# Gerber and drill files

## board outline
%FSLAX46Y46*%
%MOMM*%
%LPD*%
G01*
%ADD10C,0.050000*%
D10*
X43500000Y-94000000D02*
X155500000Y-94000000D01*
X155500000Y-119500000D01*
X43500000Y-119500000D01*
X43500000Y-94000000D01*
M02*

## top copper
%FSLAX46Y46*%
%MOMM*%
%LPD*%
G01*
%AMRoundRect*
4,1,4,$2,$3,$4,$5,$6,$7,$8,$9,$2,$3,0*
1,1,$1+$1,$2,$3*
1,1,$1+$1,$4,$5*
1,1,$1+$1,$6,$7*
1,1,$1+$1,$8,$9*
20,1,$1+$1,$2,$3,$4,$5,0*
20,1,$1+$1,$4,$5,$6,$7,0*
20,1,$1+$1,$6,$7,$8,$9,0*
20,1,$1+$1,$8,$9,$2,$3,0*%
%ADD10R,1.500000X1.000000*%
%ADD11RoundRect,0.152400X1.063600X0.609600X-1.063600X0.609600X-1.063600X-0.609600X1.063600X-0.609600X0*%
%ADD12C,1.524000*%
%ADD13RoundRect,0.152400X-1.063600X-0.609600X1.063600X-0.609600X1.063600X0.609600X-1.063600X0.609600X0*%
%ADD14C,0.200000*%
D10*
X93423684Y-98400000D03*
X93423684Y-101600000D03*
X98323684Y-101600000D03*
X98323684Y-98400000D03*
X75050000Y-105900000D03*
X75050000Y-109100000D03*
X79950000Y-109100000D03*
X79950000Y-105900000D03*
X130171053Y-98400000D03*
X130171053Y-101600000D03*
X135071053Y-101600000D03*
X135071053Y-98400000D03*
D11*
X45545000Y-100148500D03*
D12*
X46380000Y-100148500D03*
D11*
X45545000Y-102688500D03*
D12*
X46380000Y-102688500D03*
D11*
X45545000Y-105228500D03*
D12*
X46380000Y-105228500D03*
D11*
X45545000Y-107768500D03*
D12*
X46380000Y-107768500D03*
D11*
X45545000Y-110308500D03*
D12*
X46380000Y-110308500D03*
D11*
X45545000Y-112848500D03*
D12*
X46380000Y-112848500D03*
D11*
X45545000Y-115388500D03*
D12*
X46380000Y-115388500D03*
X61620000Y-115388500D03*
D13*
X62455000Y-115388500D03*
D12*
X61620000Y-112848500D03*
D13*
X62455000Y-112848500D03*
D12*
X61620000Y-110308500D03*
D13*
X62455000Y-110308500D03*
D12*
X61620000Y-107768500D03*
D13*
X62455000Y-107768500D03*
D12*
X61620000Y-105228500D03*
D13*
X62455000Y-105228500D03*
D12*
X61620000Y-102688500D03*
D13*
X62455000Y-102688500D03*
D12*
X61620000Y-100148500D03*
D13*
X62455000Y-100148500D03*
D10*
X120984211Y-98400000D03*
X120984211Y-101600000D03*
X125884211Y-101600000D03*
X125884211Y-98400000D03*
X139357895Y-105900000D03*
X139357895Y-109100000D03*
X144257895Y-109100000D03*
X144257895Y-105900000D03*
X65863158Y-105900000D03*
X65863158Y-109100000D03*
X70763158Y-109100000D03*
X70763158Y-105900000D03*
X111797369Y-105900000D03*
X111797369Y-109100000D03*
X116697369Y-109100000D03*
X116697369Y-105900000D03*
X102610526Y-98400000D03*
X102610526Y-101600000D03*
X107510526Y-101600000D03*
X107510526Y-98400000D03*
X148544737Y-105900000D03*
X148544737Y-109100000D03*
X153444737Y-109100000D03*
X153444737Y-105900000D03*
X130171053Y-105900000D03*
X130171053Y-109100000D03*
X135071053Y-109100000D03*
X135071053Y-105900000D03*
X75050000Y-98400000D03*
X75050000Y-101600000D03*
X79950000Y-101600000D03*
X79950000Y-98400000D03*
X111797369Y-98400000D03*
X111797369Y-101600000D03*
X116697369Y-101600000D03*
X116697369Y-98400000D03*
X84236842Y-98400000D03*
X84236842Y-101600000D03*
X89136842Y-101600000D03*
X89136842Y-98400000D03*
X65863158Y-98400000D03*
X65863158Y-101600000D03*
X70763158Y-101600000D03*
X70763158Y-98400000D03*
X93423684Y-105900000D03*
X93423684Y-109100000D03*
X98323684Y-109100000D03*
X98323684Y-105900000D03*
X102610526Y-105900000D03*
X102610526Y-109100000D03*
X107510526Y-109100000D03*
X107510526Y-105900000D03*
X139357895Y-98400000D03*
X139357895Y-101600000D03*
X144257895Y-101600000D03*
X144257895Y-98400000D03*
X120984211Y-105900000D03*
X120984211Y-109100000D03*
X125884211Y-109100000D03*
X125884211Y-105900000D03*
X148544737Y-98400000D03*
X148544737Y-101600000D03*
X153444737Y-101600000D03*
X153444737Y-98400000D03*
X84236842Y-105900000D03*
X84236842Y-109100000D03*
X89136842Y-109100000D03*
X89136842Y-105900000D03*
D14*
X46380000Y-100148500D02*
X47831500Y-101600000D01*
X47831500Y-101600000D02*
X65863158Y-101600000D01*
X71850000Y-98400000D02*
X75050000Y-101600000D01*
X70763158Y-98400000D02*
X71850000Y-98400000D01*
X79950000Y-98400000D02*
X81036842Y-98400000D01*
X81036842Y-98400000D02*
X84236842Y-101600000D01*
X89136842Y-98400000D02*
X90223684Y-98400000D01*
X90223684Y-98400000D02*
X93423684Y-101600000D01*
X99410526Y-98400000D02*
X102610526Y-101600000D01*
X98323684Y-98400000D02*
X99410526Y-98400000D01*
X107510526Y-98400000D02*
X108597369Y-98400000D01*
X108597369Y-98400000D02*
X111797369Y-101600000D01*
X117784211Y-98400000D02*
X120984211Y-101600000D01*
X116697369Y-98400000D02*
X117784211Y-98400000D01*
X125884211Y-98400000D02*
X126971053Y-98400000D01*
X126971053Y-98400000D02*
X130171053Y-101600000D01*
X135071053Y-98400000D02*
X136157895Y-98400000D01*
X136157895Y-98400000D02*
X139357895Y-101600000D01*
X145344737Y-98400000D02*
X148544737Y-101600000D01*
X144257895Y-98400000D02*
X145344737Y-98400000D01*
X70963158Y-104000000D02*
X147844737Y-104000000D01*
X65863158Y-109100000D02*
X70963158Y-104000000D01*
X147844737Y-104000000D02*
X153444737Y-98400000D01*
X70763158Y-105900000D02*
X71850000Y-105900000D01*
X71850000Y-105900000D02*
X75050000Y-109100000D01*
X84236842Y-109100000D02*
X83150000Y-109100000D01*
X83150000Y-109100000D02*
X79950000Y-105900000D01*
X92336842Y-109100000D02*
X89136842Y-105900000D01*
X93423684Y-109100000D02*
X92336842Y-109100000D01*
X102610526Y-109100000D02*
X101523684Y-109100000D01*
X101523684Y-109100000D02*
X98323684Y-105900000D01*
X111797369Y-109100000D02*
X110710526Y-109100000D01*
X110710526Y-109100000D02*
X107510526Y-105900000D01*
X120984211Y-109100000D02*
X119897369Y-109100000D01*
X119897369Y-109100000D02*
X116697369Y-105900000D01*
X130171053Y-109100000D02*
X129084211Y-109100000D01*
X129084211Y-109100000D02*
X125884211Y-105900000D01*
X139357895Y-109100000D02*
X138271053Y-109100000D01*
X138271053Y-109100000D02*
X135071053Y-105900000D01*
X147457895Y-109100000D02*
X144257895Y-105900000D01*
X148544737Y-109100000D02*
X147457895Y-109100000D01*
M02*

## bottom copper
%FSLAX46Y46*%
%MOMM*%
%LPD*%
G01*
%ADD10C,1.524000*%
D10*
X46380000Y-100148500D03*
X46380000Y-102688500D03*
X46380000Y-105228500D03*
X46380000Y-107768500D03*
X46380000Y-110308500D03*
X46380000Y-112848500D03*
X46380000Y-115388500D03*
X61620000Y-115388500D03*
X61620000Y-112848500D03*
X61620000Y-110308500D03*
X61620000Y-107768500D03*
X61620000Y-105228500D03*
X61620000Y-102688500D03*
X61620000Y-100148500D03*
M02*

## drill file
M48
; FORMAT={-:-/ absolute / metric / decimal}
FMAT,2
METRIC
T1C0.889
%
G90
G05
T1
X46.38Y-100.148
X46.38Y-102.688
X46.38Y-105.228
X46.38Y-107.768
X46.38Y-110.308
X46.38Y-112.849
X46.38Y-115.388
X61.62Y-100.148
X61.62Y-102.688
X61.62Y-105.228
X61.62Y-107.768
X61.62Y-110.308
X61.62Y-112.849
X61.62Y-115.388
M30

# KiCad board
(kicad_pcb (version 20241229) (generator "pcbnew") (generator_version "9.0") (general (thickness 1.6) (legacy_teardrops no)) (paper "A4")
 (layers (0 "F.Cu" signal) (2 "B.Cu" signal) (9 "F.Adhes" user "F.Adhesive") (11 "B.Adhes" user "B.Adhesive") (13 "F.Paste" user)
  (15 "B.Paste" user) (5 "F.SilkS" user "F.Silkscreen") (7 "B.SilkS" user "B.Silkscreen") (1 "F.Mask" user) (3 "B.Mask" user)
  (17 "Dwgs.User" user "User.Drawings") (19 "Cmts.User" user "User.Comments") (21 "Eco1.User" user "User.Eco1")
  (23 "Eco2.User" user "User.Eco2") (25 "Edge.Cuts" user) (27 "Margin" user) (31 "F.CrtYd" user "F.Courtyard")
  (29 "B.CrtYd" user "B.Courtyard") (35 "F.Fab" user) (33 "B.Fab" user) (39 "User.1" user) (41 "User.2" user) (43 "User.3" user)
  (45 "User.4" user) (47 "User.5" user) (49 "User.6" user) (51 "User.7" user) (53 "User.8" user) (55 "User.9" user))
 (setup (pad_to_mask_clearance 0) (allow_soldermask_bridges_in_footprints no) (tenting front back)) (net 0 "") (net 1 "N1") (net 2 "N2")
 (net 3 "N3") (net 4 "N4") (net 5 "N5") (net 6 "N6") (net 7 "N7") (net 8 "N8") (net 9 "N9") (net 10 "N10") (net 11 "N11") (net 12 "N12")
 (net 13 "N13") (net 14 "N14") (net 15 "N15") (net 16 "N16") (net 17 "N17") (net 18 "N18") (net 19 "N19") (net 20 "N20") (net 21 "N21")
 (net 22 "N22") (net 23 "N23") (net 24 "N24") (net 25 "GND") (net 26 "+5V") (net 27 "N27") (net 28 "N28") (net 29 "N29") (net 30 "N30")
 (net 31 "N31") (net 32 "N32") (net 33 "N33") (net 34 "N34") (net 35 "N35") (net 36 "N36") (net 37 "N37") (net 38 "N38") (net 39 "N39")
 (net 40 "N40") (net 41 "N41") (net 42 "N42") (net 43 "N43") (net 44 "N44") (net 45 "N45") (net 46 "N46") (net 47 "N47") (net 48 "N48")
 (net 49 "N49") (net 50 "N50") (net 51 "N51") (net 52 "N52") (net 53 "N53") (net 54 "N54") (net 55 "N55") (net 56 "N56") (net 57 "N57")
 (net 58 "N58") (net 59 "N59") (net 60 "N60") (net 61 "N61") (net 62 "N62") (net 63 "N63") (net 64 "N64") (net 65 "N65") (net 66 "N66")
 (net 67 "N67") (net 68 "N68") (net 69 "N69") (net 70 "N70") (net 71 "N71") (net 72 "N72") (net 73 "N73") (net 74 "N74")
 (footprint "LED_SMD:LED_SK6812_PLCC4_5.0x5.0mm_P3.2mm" (layer "F.Cu") (at 95.873684 100)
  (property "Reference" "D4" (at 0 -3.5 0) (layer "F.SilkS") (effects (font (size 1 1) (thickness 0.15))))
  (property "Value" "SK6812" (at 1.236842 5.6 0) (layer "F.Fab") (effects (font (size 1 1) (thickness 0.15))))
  (pad "1" smd rect (at -2.45 -1.6 180) (size 1.5 1) (layers "F.Cu" "F.Mask" "F.Paste") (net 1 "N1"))
  (pad "2" smd rect (at -2.45 1.6 180) (size 1.5 1) (layers "F.Cu" "F.Mask" "F.Paste") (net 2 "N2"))
  (pad "3" smd rect (at 2.45 1.6 180) (size 1.5 1) (layers "F.Cu" "F.Mask" "F.Paste") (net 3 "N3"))
  (pad "4" smd rect (at 2.45 -1.6 180) (size 1.5 1) (layers "F.Cu" "F.Mask" "F.Paste") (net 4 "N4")))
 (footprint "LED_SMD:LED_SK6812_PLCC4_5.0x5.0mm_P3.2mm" (layer "F.Cu") (at 77.5 107.5)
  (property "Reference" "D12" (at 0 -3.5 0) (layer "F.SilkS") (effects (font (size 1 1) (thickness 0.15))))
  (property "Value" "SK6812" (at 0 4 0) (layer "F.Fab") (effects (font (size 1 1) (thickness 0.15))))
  (pad "1" smd rect (at -2.45 -1.6 180) (size 1.5 1) (layers "F.Cu" "F.Mask" "F.Paste") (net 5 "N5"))
  (pad "2" smd rect (at -2.45 1.6 180) (size 1.5 1) (layers "F.Cu" "F.Mask" "F.Paste") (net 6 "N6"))
  (pad "3" smd rect (at 2.45 1.6 180) (size 1.5 1) (layers "F.Cu" "F.Mask" "F.Paste") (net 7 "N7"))
  (pad "4" smd rect (at 2.45 -1.6 180) (size 1.5 1) (layers "F.Cu" "F.Mask" "F.Paste") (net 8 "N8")))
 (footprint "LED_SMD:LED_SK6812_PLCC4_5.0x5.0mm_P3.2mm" (layer "F.Cu") (at 132.621053 100)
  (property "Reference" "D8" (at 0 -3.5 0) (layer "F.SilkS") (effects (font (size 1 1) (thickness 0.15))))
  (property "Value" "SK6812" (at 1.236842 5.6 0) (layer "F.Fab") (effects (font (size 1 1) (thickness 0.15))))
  (pad "1" smd rect (at -2.45 -1.6 180) (size 1.5 1) (layers "F.Cu" "F.Mask" "F.Paste") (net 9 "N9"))
  (pad "2" smd rect (at -2.45 1.6 180) (size 1.5 1) (layers "F.Cu" "F.Mask" "F.Paste") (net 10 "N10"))
  (pad "3" smd rect (at 2.45 1.6 180) (size 1.5 1) (layers "F.Cu" "F.Mask" "F.Paste") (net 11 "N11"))
  (pad "4" smd rect (at 2.45 -1.6 180) (size 1.5 1) (layers "F.Cu" "F.Mask" "F.Paste") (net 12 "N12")))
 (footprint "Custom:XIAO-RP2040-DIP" (layer "F.Cu") (at 54 107.7685)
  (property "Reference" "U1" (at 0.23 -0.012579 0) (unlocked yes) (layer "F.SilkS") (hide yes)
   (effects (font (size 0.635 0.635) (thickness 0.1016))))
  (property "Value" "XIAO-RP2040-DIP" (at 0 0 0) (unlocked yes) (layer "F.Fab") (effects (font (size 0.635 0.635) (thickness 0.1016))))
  (pad "1" smd roundrect (at -8.455 -7.62 180) (size 2.432 1.524) (layers "F.Cu" "F.Mask") (roundrect_rratio 0.1) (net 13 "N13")
   (thermal_bridge_angle 45))
  (pad "1" thru_hole circle (at -7.62 -7.62 180) (size 1.524 1.524) (drill 0.889) (layers "*.Cu" "*.Mask") (remove_unused_layers no)
   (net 13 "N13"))
  (pad "2" smd roundrect (at -8.455 -5.08 180) (size 2.432 1.524) (layers "F.Cu" "F.Mask") (roundrect_rratio 0.1) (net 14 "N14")
   (thermal_bridge_angle 45))
  (pad "2" thru_hole circle (at -7.62 -5.08 180) (size 1.524 1.524) (drill 0.889) (layers "*.Cu" "*.Mask") (remove_unused_layers no)
   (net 14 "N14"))
  (pad "3" smd roundrect (at -8.455 -2.54 180) (size 2.432 1.524) (layers "F.Cu" "F.Mask") (roundrect_rratio 0.1) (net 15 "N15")
   (thermal_bridge_angle 45))
  (pad "3" thru_hole circle (at -7.62 -2.54 180) (size 1.524 1.524) (drill 0.889) (layers "*.Cu" "*.Mask") (remove_unused_layers no)
   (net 15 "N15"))
  (pad "4" smd roundrect (at -8.455 0 180) (size 2.432 1.524) (layers "F.Cu" "F.Mask") (roundrect_rratio 0.1) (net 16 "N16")
   (thermal_bridge_angle 45))
  (pad "4" thru_hole circle (at -7.62 0 180) (size 1.524 1.524) (drill 0.889) (layers "*.Cu" "*.Mask") (remove_unused_layers no)
   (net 16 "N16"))
  (pad "5" smd roundrect (at -8.455 2.54 180) (size 2.432 1.524) (layers "F.Cu" "F.Mask") (roundrect_rratio 0.1) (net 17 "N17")
   (thermal_bridge_angle 45))
  (pad "5" thru_hole circle (at -7.62 2.54 180) (size 1.524 1.524) (drill 0.889) (layers "*.Cu" "*.Mask") (remove_unused_layers no)
   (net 17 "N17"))
  (pad "6" smd roundrect (at -8.455 5.08 180) (size 2.432 1.524) (layers "F.Cu" "F.Mask") (roundrect_rratio 0.1) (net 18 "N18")
   (thermal_bridge_angle 45))
  (pad "6" thru_hole circle (at -7.62 5.08 180) (size 1.524 1.524) (drill 0.889) (layers "*.Cu" "*.Mask") (remove_unused_layers no)
   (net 18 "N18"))
  (pad "7" smd roundrect (at -8.455 7.62 180) (size 2.432 1.524) (layers "F.Cu" "F.Mask") (roundrect_rratio 0.1) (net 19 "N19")
   (thermal_bridge_angle 45))
  (pad "7" thru_hole circle (at -7.62 7.62 180) (size 1.524 1.524) (drill 0.889) (layers "*.Cu" "*.Mask") (remove_unused_layers no)
   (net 19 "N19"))
  (pad "8" thru_hole circle (at 7.62 7.62) (size 1.524 1.524) (drill 0.889) (layers "*.Cu" "*.Mask") (remove_unused_layers no)
   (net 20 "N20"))
  (pad "8" smd roundrect (at 8.455 7.62) (size 2.432 1.524) (layers "F.Cu" "F.Mask") (roundrect_rratio 0.1) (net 20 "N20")
   (thermal_bridge_angle 45))
  (pad "9" thru_hole circle (at 7.62 5.08) (size 1.524 1.524) (drill 0.889) (layers "*.Cu" "*.Mask") (remove_unused_layers no)
   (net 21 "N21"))
  (pad "9" smd roundrect (at 8.455 5.08) (size 2.432 1.524) (layers "F.Cu" "F.Mask") (roundrect_rratio 0.1) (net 21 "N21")
   (thermal_bridge_angle 45))
  (pad "10" thru_hole circle (at 7.62 2.54) (size 1.524 1.524) (drill 0.889) (layers "*.Cu" "*.Mask") (remove_unused_layers no)
   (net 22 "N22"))
  (pad "10" smd roundrect (at 8.455 2.54) (size 2.432 1.524) (layers "F.Cu" "F.Mask") (roundrect_rratio 0.1) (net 22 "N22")
   (thermal_bridge_angle 45))
  (pad "11" thru_hole circle (at 7.62 0) (size 1.524 1.524) (drill 0.889) (layers "*.Cu" "*.Mask") (remove_unused_layers no) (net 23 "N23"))
  (pad "11" smd roundrect (at 8.455 0) (size 2.432 1.524) (layers "F.Cu" "F.Mask") (roundrect_rratio 0.1) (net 23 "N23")
   (thermal_bridge_angle 45))
  (pad "12" thru_hole circle (at 7.62 -2.54) (size 1.524 1.524) (drill 0.889) (layers "*.Cu" "*.Mask") (remove_unused_layers no)
   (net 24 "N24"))
  (pad "12" smd roundrect (at 8.455 -2.54) (size 2.432 1.524) (layers "F.Cu" "F.Mask") (roundrect_rratio 0.1) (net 24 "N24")
   (thermal_bridge_angle 45))
  (pad "13" thru_hole circle (at 7.62 -5.08) (size 1.524 1.524) (drill 0.889) (layers "*.Cu" "*.Mask") (remove_unused_layers no)
   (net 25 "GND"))
  (pad "13" smd roundrect (at 8.455 -5.08) (size 2.432 1.524) (layers "F.Cu" "F.Mask") (roundrect_rratio 0.1) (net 25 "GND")
   (thermal_bridge_angle 45))
  (pad "14" thru_hole circle (at 7.62 -7.62) (size 1.524 1.524) (drill 0.889) (layers "*.Cu" "*.Mask") (remove_unused_layers no)
   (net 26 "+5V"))
  (pad "14" smd roundrect (at 8.455 -7.62) (size 2.432 1.524) (layers "F.Cu" "F.Mask") (roundrect_rratio 0.1) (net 26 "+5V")
   (thermal_bridge_angle 45)))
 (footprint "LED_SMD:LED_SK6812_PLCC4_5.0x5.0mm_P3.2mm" (layer "F.Cu") (at 123.434211 100)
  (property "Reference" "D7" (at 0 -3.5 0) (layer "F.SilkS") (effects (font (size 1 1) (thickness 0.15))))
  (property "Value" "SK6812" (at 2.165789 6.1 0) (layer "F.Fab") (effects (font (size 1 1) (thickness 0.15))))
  (pad "1" smd rect (at -2.45 -1.6 180) (size 1.5 1) (layers "F.Cu" "F.Mask" "F.Paste") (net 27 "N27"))
  (pad "2" smd rect (at -2.45 1.6 180) (size 1.5 1) (layers "F.Cu" "F.Mask" "F.Paste") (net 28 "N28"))
  (pad "3" smd rect (at 2.45 1.6 180) (size 1.5 1) (layers "F.Cu" "F.Mask" "F.Paste") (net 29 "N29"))
  (pad "4" smd rect (at 2.45 -1.6 180) (size 1.5 1) (layers "F.Cu" "F.Mask" "F.Paste") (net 10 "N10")))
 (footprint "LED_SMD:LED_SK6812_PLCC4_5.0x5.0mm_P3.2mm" (layer "F.Cu") (at 141.807895 107.5)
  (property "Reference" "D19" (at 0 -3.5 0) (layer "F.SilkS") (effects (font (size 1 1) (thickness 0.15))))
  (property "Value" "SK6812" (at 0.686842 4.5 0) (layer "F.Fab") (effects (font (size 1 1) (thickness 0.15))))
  (pad "1" smd rect (at -2.45 -1.6 180) (size 1.5 1) (layers "F.Cu" "F.Mask" "F.Paste") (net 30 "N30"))
  (pad "2" smd rect (at -2.45 1.6 180) (size 1.5 1) (layers "F.Cu" "F.Mask" "F.Paste") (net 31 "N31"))
  (pad "3" smd rect (at 2.45 1.6 180) (size 1.5 1) (layers "F.Cu" "F.Mask" "F.Paste") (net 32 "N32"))
  (pad "4" smd rect (at 2.45 -1.6 180) (size 1.5 1) (layers "F.Cu" "F.Mask" "F.Paste") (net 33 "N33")))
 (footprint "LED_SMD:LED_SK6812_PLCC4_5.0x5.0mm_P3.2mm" (layer "F.Cu") (at 68.313158 107.5)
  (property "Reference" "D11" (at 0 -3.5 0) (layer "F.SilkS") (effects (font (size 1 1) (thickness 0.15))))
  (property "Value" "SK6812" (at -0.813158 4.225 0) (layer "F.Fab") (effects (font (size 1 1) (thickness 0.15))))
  (pad "1" smd rect (at -2.45 -1.6 180) (size 1.5 1) (layers "F.Cu" "F.Mask" "F.Paste") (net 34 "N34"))
  (pad "2" smd rect (at -2.45 1.6 180) (size 1.5 1) (layers "F.Cu" "F.Mask" "F.Paste") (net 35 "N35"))
  (pad "3" smd rect (at 2.45 1.6 180) (size 1.5 1) (layers "F.Cu" "F.Mask" "F.Paste") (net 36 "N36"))
  (pad "4" smd rect (at 2.45 -1.6 180) (size 1.5 1) (layers "F.Cu" "F.Mask" "F.Paste") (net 6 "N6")))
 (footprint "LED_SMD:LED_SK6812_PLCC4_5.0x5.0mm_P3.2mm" (layer "F.Cu") (at 114.247369 107.5)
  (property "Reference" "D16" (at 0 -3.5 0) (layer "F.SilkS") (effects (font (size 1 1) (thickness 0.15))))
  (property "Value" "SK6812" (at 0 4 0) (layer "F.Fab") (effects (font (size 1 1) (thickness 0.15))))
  (pad "1" smd rect (at -2.45 -1.6 180) (size 1.5 1) (layers "F.Cu" "F.Mask" "F.Paste") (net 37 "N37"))
  (pad "2" smd rect (at -2.45 1.6 180) (size 1.5 1) (layers "F.Cu" "F.Mask" "F.Paste") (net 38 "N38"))
  (pad "3" smd rect (at 2.45 1.6 180) (size 1.5 1) (layers "F.Cu" "F.Mask" "F.Paste") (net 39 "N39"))
  (pad "4" smd rect (at 2.45 -1.6 180) (size 1.5 1) (layers "F.Cu" "F.Mask" "F.Paste") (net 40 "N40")))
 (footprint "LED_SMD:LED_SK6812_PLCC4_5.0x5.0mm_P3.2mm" (layer "F.Cu") (at 105.060526 100)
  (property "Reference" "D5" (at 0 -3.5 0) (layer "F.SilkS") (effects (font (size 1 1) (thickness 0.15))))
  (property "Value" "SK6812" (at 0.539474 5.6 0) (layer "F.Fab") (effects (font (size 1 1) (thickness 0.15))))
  (pad "1" smd rect (at -2.45 -1.6 180) (size 1.5 1) (layers "F.Cu" "F.Mask" "F.Paste") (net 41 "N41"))
  (pad "2" smd rect (at -2.45 1.6 180) (size 1.5 1) (layers "F.Cu" "F.Mask" "F.Paste") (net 4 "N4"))
  (pad "3" smd rect (at 2.45 1.6 180) (size 1.5 1) (layers "F.Cu" "F.Mask" "F.Paste") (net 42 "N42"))
  (pad "4" smd rect (at 2.45 -1.6 180) (size 1.5 1) (layers "F.Cu" "F.Mask" "F.Paste") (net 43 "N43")))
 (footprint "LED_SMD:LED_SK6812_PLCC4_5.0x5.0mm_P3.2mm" (layer "F.Cu") (at 150.994737 107.5)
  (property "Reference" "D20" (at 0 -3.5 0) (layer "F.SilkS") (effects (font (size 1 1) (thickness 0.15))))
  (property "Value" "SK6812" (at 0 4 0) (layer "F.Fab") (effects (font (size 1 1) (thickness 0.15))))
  (pad "1" smd rect (at -2.45 -1.6 180) (size 1.5 1) (layers "F.Cu" "F.Mask" "F.Paste") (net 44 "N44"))
  (pad "2" smd rect (at -2.45 1.6 180) (size 1.5 1) (layers "F.Cu" "F.Mask" "F.Paste") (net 33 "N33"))
  (pad "3" smd rect (at 2.45 1.6 180) (size 1.5 1) (layers "F.Cu" "F.Mask" "F.Paste") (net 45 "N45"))
  (pad "4" smd rect (at 2.45 -1.6 180) (size 1.5 1) (layers "F.Cu" "F.Mask" "F.Paste") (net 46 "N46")))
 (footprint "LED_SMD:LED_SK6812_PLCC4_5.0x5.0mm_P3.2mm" (layer "F.Cu") (at 132.621053 107.5)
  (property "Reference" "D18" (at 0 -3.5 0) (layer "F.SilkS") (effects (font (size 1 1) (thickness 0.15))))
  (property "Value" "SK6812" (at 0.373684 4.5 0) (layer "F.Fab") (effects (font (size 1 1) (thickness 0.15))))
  (pad "1" smd rect (at -2.45 -1.6 180) (size 1.5 1) (layers "F.Cu" "F.Mask" "F.Paste") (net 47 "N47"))
  (pad "2" smd rect (at -2.45 1.6 180) (size 1.5 1) (layers "F.Cu" "F.Mask" "F.Paste") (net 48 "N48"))
  (pad "3" smd rect (at 2.45 1.6 180) (size 1.5 1) (layers "F.Cu" "F.Mask" "F.Paste") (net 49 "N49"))
  (pad "4" smd rect (at 2.45 -1.6 180) (size 1.5 1) (layers "F.Cu" "F.Mask" "F.Paste") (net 31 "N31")))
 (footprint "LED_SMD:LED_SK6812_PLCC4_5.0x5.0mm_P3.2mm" (layer "F.Cu") (at 77.5 100)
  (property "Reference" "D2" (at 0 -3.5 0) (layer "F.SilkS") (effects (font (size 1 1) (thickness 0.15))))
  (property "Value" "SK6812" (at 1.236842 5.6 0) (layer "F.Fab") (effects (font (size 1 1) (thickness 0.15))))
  (pad "1" smd rect (at -2.45 -1.6 180) (size 1.5 1) (layers "F.Cu" "F.Mask" "F.Paste") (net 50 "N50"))
  (pad "2" smd rect (at -2.45 1.6 180) (size 1.5 1) (layers "F.Cu" "F.Mask" "F.Paste") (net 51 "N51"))
  (pad "3" smd rect (at 2.45 1.6 180) (size 1.5 1) (layers "F.Cu" "F.Mask" "F.Paste") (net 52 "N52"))
  (pad "4" smd rect (at 2.45 -1.6 180) (size 1.5 1) (layers "F.Cu" "F.Mask" "F.Paste") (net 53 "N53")))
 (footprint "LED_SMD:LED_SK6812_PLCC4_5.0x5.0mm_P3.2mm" (layer "F.Cu") (at 114.247369 100)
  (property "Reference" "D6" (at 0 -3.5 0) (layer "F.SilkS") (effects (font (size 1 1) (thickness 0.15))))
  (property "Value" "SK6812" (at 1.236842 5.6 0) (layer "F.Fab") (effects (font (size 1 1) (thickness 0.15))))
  (pad "1" smd rect (at -2.45 -1.6 180) (size 1.5 1) (layers "F.Cu" "F.Mask" "F.Paste") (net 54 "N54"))
  (pad "2" smd rect (at -2.45 1.6 180) (size 1.5 1) (layers "F.Cu" "F.Mask" "F.Paste") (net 43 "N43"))
  (pad "3" smd rect (at 2.45 1.6 180) (size 1.5 1) (layers "F.Cu" "F.Mask" "F.Paste") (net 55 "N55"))
  (pad "4" smd rect (at 2.45 -1.6 180) (size 1.5 1) (layers "F.Cu" "F.Mask" "F.Paste") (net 28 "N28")))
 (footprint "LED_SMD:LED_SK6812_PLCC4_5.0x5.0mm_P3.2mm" (layer "F.Cu") (at 86.686842 100)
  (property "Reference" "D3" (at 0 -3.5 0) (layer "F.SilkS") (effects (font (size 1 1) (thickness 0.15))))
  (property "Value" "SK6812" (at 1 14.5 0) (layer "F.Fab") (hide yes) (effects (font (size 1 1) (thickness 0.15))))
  (pad "1" smd rect (at -2.45 -1.6 180) (size 1.5 1) (layers "F.Cu" "F.Mask" "F.Paste") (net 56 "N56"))
  (pad "2" smd rect (at -2.45 1.6 180) (size 1.5 1) (layers "F.Cu" "F.Mask" "F.Paste") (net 53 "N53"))
  (pad "3" smd rect (at 2.45 1.6 180) (size 1.5 1) (layers "F.Cu" "F.Mask" "F.Paste") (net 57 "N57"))
  (pad "4" smd rect (at 2.45 -1.6 180) (size 1.5 1) (layers "F.Cu" "F.Mask" "F.Paste") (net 2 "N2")))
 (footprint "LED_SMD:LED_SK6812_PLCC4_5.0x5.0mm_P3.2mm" (layer "F.Cu") (at 68.313158 100)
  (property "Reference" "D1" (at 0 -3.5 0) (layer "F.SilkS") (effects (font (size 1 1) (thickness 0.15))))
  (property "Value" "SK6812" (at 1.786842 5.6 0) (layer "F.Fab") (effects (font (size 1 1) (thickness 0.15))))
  (pad "1" smd rect (at -2.45 -1.6 180) (size 1.5 1) (layers "F.Cu" "F.Mask" "F.Paste") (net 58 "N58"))
  (pad "2" smd rect (at -2.45 1.6 180) (size 1.5 1) (layers "F.Cu" "F.Mask" "F.Paste") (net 13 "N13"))
  (pad "3" smd rect (at 2.45 1.6 180) (size 1.5 1) (layers "F.Cu" "F.Mask" "F.Paste") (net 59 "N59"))
  (pad "4" smd rect (at 2.45 -1.6 180) (size 1.5 1) (layers "F.Cu" "F.Mask" "F.Paste") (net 51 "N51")))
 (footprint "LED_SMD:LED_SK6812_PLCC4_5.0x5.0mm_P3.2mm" (layer "F.Cu") (at 95.873684 107.5)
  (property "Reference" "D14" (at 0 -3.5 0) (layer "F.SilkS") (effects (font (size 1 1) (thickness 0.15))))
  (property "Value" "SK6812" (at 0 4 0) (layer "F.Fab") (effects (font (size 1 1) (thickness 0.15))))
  (pad "1" smd rect (at -2.45 -1.6 180) (size 1.5 1) (layers "F.Cu" "F.Mask" "F.Paste") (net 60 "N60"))
  (pad "2" smd rect (at -2.45 1.6 180) (size 1.5 1) (layers "F.Cu" "F.Mask" "F.Paste") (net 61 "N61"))
  (pad "3" smd rect (at 2.45 1.6 180) (size 1.5 1) (layers "F.Cu" "F.Mask" "F.Paste") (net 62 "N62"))
  (pad "4" smd rect (at 2.45 -1.6 180) (size 1.5 1) (layers "F.Cu" "F.Mask" "F.Paste") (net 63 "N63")))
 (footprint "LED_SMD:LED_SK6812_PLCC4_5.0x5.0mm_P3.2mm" (layer "F.Cu") (at 105.060526 107.5)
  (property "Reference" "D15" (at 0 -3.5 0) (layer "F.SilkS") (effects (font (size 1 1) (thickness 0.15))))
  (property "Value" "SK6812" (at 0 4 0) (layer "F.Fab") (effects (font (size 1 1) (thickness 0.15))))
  (pad "1" smd rect (at -2.45 -1.6 180) (size 1.5 1) (layers "F.Cu" "F.Mask" "F.Paste") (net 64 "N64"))
  (pad "2" smd rect (at -2.45 1.6 180) (size 1.5 1) (layers "F.Cu" "F.Mask" "F.Paste") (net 63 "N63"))
  (pad "3" smd rect (at 2.45 1.6 180) (size 1.5 1) (layers "F.Cu" "F.Mask" "F.Paste") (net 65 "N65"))
  (pad "4" smd rect (at 2.45 -1.6 180) (size 1.5 1) (layers "F.Cu" "F.Mask" "F.Paste") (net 38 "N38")))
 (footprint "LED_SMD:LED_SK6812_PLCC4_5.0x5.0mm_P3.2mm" (layer "F.Cu") (at 141.807895 100)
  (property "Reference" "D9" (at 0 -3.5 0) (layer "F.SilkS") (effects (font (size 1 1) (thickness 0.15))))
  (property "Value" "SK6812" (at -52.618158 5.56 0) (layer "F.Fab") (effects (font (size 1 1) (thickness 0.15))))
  (pad "1" smd rect (at -2.45 -1.6 180) (size 1.5 1) (layers "F.Cu" "F.Mask" "F.Paste") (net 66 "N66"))
  (pad "2" smd rect (at -2.45 1.6 180) (size 1.5 1) (layers "F.Cu" "F.Mask" "F.Paste") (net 12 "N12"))
  (pad "3" smd rect (at 2.45 1.6 180) (size 1.5 1) (layers "F.Cu" "F.Mask" "F.Paste") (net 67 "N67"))
  (pad "4" smd rect (at 2.45 -1.6 180) (size 1.5 1) (layers "F.Cu" "F.Mask" "F.Paste") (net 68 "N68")))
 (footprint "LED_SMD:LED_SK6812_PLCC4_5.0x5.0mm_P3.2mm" (layer "F.Cu") (at 123.434211 107.5)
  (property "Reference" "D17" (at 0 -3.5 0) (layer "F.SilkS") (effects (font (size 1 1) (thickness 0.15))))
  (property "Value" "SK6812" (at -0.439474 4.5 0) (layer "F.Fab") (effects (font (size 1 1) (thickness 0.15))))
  (pad "1" smd rect (at -2.45 -1.6 180) (size 1.5 1) (layers "F.Cu" "F.Mask" "F.Paste") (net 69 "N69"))
  (pad "2" smd rect (at -2.45 1.6 180) (size 1.5 1) (layers "F.Cu" "F.Mask" "F.Paste") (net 40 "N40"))
  (pad "3" smd rect (at 2.45 1.6 180) (size 1.5 1) (layers "F.Cu" "F.Mask" "F.Paste") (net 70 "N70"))
  (pad "4" smd rect (at 2.45 -1.6 180) (size 1.5 1) (layers "F.Cu" "F.Mask" "F.Paste") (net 48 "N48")))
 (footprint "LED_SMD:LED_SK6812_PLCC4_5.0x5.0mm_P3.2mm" (layer "F.Cu") (at 150.994737 100)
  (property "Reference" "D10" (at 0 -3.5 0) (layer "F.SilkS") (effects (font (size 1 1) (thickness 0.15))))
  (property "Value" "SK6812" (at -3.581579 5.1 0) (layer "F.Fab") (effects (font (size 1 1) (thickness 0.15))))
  (pad "1" smd rect (at -2.45 -1.6 180) (size 1.5 1) (layers "F.Cu" "F.Mask" "F.Paste") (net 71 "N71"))
  (pad "2" smd rect (at -2.45 1.6 180) (size 1.5 1) (layers "F.Cu" "F.Mask" "F.Paste") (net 68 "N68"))
  (pad "3" smd rect (at 2.45 1.6 180) (size 1.5 1) (layers "F.Cu" "F.Mask" "F.Paste") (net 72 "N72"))
  (pad "4" smd rect (at 2.45 -1.6 180) (size 1.5 1) (layers "F.Cu" "F.Mask" "F.Paste") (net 35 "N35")))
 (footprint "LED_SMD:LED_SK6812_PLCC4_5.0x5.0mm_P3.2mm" (layer "F.Cu") (at 86.686842 107.5)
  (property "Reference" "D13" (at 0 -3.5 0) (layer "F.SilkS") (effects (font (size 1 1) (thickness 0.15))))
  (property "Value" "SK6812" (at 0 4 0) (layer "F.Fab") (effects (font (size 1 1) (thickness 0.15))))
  (pad "1" smd rect (at -2.45 -1.6 180) (size 1.5 1) (layers "F.Cu" "F.Mask" "F.Paste") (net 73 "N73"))
  (pad "2" smd rect (at -2.45 1.6 180) (size 1.5 1) (layers "F.Cu" "F.Mask" "F.Paste") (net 8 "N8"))
  (pad "3" smd rect (at 2.45 1.6 180) (size 1.5 1) (layers "F.Cu" "F.Mask" "F.Paste") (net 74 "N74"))
  (pad "4" smd rect (at 2.45 -1.6 180) (size 1.5 1) (layers "F.Cu" "F.Mask" "F.Paste") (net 61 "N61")))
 (gr_rect (start 43.5 94) (end 155.5 119.5) (stroke (width 0.05) (type default)) (fill no) (layer "Edge.Cuts"))
 (segment (start 46.38 100.1485) (end 47.8315 101.6) (width 0.2) (layer "F.Cu") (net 13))
 (segment (start 47.8315 101.6) (end 65.863158 101.6) (width 0.2) (layer "F.Cu") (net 13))
 (segment (start 71.85 98.4) (end 75.05 101.6) (width 0.2) (layer "F.Cu") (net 51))
 (segment (start 70.763158 98.4) (end 71.85 98.4) (width 0.2) (layer "F.Cu") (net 51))
 (segment (start 79.95 98.4) (end 81.036842 98.4) (width 0.2) (layer "F.Cu") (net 53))
 (segment (start 81.036842 98.4) (end 84.236842 101.6) (width 0.2) (layer "F.Cu") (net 53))
 (segment (start 89.136842 98.4) (end 90.223684 98.4) (width 0.2) (layer "F.Cu") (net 2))
 (segment (start 90.223684 98.4) (end 93.423684 101.6) (width 0.2) (layer "F.Cu") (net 2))
 (segment (start 99.410526 98.4) (end 102.610526 101.6) (width 0.2) (layer "F.Cu") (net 4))
 (segment (start 98.323684 98.4) (end 99.410526 98.4) (width 0.2) (layer "F.Cu") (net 4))
 (segment (start 107.510526 98.4) (end 108.597369 98.4) (width 0.2) (layer "F.Cu") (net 43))
 (segment (start 108.597369 98.4) (end 111.797369 101.6) (width 0.2) (layer "F.Cu") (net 43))
 (segment (start 117.784211 98.4) (end 120.984211 101.6) (width 0.2) (layer "F.Cu") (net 28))
 (segment (start 116.697369 98.4) (end 117.784211 98.4) (width 0.2) (layer "F.Cu") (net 28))
 (segment (start 125.884211 98.4) (end 126.971053 98.4) (width 0.2) (layer "F.Cu") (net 10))
 (segment (start 126.971053 98.4) (end 130.171053 101.6) (width 0.2) (layer "F.Cu") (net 10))
 (segment (start 135.071053 98.4) (end 136.157895 98.4) (width 0.2) (layer "F.Cu") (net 12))
 (segment (start 136.157895 98.4) (end 139.357895 101.6) (width 0.2) (layer "F.Cu") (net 12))
 (segment (start 145.344737 98.4) (end 148.544737 101.6) (width 0.2) (layer "F.Cu") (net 68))
 (segment (start 144.257895 98.4) (end 145.344737 98.4) (width 0.2) (layer "F.Cu") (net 68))
 (segment (start 70.963158 104) (end 147.844737 104) (width 0.2) (layer "F.Cu") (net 35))
 (segment (start 65.863158 109.1) (end 70.963158 104) (width 0.2) (layer "F.Cu") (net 35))
 (segment (start 147.844737 104) (end 153.444737 98.4) (width 0.2) (layer "F.Cu") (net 35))
 (segment (start 70.763158 105.9) (end 71.85 105.9) (width 0.2) (layer "F.Cu") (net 6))
 (segment (start 71.85 105.9) (end 75.05 109.1) (width 0.2) (layer "F.Cu") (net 6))
 (segment (start 84.236842 109.1) (end 83.15 109.1) (width 0.2) (layer "F.Cu") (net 8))
 (segment (start 83.15 109.1) (end 79.95 105.9) (width 0.2) (layer "F.Cu") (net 8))
 (segment (start 92.336842 109.1) (end 89.136842 105.9) (width 0.2) (layer "F.Cu") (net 61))
 (segment (start 93.423684 109.1) (end 92.336842 109.1) (width 0.2) (layer "F.Cu") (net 61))
 (segment (start 102.610526 109.1) (end 101.523684 109.1) (width 0.2) (layer "F.Cu") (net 63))
 (segment (start 101.523684 109.1) (end 98.323684 105.9) (width 0.2) (layer "F.Cu") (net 63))
 (segment (start 111.797369 109.1) (end 110.710526 109.1) (width 0.2) (layer "F.Cu") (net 38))
 (segment (start 110.710526 109.1) (end 107.510526 105.9) (width 0.2) (layer "F.Cu") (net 38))
 (segment (start 120.984211 109.1) (end 119.897369 109.1) (width 0.2) (layer "F.Cu") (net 40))
 (segment (start 119.897369 109.1) (end 116.697369 105.9) (width 0.2) (layer "F.Cu") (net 40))
 (segment (start 130.171053 109.1) (end 129.084211 109.1) (width 0.2) (layer "F.Cu") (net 48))
 (segment (start 129.084211 109.1) (end 125.884211 105.9) (width 0.2) (layer "F.Cu") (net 48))
 (segment (start 139.357895 109.1) (end 138.271053 109.1) (width 0.2) (layer "F.Cu") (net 31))
 (segment (start 138.271053 109.1) (end 135.071053 105.9) (width 0.2) (layer "F.Cu") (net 31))
 (segment (start 147.457895 109.1) (end 144.257895 105.9) (width 0.2) (layer "F.Cu") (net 33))
 (segment (start 148.544737 109.1) (end 147.457895 109.1) (width 0.2) (layer "F.Cu") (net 33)))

